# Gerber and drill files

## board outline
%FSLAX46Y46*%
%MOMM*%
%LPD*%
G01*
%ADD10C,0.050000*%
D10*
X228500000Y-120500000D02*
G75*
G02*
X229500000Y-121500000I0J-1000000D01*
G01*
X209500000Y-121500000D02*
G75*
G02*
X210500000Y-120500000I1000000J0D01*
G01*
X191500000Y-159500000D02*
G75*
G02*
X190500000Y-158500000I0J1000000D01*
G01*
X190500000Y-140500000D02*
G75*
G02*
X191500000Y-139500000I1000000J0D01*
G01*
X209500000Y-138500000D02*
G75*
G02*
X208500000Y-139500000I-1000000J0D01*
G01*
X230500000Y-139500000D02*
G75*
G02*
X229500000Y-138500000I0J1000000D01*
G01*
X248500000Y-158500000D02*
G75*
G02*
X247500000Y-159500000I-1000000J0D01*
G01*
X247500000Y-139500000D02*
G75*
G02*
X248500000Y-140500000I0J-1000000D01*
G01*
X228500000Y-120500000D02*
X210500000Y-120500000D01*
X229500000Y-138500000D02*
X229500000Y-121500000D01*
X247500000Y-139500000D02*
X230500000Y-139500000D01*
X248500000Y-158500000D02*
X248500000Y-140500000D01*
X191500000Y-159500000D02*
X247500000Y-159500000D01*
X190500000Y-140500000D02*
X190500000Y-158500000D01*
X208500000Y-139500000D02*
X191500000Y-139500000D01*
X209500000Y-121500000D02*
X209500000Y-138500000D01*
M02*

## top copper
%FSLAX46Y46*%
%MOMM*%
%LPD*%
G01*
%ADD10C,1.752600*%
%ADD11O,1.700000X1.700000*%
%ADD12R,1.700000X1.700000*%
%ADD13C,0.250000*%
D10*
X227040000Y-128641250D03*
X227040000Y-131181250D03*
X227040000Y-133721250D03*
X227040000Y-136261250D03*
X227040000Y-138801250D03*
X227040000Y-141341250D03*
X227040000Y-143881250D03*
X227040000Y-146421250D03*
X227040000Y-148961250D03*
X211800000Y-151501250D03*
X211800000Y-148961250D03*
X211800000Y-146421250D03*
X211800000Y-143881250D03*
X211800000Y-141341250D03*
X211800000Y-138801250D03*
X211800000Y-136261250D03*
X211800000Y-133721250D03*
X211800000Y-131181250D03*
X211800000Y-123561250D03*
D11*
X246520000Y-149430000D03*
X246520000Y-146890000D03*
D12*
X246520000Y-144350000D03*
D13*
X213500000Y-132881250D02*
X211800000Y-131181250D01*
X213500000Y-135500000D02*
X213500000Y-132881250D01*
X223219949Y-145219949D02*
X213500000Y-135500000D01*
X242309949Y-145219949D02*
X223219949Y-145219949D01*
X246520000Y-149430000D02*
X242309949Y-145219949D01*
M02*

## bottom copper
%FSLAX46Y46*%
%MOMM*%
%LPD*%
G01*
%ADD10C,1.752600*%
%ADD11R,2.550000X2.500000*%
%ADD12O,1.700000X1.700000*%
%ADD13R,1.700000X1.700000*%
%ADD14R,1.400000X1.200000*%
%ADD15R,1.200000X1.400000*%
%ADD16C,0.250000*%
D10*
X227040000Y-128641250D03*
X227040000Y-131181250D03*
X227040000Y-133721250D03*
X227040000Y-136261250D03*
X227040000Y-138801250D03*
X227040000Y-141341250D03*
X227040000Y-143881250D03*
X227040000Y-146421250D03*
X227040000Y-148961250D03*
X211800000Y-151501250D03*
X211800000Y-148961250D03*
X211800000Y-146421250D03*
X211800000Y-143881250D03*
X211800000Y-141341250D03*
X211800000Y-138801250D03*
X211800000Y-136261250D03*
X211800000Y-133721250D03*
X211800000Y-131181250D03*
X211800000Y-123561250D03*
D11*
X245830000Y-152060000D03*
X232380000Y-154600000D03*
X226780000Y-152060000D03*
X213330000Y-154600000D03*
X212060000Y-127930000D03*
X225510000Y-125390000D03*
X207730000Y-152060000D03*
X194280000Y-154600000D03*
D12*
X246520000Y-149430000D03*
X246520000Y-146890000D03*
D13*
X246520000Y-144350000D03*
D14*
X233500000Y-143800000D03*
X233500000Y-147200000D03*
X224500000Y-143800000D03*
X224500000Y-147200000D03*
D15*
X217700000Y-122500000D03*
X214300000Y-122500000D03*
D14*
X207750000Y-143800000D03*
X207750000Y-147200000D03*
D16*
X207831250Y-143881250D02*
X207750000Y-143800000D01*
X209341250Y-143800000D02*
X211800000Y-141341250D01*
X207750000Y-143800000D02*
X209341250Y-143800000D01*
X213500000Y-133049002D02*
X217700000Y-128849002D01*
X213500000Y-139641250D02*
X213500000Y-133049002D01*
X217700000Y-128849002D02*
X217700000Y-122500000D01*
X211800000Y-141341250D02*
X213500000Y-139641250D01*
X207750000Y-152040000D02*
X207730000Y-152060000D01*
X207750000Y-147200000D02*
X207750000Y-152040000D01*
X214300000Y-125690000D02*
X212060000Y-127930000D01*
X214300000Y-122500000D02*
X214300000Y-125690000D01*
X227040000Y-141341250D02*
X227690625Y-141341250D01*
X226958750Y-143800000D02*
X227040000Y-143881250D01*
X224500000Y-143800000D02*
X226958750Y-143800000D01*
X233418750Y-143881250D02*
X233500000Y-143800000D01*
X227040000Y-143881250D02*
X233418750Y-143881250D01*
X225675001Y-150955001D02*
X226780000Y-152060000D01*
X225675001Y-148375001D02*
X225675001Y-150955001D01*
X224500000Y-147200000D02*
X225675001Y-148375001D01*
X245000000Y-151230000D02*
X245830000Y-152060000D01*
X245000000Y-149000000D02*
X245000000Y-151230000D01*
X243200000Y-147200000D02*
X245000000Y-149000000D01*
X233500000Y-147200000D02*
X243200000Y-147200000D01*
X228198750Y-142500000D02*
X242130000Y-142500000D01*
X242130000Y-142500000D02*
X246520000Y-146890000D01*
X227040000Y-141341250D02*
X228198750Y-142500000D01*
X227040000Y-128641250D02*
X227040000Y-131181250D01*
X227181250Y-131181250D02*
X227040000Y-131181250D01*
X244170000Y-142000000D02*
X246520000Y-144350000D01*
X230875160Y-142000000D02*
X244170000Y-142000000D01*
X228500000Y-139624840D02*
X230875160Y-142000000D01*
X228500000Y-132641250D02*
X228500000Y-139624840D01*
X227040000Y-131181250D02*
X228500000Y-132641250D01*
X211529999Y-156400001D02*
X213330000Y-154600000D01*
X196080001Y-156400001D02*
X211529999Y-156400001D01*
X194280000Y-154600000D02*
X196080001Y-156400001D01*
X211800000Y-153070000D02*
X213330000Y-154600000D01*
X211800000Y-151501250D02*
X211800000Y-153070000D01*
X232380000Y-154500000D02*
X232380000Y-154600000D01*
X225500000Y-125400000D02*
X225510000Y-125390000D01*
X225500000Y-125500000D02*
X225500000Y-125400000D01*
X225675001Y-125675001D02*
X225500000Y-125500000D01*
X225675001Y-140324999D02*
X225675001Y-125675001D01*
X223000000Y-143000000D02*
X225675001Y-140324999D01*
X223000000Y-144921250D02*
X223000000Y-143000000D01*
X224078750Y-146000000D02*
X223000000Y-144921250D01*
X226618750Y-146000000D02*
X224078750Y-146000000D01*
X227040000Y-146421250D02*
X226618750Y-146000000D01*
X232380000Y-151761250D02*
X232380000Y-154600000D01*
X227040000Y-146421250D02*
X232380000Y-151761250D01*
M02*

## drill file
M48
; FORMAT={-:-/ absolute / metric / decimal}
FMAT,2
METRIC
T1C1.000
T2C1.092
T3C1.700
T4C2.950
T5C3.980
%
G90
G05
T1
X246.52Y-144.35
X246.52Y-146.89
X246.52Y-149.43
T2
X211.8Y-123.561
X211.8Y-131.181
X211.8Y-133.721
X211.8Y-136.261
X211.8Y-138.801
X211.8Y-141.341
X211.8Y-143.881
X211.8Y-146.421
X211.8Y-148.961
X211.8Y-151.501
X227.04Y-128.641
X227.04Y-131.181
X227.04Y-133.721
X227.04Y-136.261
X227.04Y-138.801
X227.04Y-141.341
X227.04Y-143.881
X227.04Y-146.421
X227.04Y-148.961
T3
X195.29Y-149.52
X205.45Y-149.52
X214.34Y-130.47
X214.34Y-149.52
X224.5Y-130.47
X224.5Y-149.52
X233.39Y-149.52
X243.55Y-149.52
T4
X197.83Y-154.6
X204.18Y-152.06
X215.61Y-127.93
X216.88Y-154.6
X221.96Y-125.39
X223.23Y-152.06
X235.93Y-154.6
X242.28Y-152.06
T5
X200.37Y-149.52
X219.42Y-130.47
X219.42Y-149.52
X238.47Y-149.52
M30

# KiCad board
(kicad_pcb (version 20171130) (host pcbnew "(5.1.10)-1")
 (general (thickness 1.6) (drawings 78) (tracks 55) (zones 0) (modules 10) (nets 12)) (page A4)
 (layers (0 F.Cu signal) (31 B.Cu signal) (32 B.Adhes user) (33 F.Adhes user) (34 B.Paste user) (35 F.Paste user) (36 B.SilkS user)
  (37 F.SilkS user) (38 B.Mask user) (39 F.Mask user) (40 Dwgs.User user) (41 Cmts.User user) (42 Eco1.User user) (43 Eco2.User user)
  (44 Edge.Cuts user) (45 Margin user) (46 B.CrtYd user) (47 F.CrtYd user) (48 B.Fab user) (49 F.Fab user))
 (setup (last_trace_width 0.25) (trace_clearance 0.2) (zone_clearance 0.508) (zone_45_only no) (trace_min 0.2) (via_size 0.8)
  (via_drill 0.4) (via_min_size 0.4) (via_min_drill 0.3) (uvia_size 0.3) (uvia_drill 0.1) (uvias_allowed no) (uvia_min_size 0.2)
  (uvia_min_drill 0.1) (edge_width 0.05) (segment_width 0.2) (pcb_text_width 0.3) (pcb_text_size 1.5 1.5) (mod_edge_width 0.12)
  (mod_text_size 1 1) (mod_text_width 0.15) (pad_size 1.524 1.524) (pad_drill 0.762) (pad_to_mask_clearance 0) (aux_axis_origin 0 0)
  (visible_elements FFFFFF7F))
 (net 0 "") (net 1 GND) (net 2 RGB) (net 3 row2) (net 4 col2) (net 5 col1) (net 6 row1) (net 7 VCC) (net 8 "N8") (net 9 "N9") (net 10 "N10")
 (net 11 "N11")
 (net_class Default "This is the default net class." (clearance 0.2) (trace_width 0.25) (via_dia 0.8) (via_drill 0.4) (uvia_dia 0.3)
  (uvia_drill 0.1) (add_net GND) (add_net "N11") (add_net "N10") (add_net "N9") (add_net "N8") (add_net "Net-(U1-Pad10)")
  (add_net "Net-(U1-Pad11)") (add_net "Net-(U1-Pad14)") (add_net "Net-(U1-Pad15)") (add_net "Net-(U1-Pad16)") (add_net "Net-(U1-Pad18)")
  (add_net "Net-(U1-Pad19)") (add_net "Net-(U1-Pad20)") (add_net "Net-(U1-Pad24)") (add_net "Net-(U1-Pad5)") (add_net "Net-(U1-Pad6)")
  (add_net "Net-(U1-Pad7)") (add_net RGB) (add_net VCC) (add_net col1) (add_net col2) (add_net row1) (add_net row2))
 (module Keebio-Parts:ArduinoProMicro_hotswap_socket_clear (layer B.Cu) (at 219.42 137.53125 270)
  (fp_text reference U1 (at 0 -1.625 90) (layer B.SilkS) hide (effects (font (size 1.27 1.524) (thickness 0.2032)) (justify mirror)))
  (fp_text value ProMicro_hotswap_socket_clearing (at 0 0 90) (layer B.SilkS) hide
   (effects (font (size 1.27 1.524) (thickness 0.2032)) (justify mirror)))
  (pad 3 thru_hole circle (at -8.89 -7.62 270) (size 1.7526 1.7526) (drill 1.0922) (layers *.Cu *.SilkS *.Mask) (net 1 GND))
  (pad 4 thru_hole circle (at -6.35 -7.62 270) (size 1.7526 1.7526) (drill 1.0922) (layers *.Cu *.SilkS *.Mask) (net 1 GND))
  (pad 5 thru_hole circle (at -3.81 -7.62 270) (size 1.7526 1.7526) (drill 1.0922) (layers *.Cu *.SilkS *.Mask))
  (pad 6 thru_hole circle (at -1.27 -7.62 270) (size 1.7526 1.7526) (drill 1.0922) (layers *.Cu *.SilkS *.Mask))
  (pad 7 thru_hole circle (at 1.27 -7.62 270) (size 1.7526 1.7526) (drill 1.0922) (layers *.Cu *.SilkS *.Mask))
  (pad 8 thru_hole circle (at 3.81 -7.62 270) (size 1.7526 1.7526) (drill 1.0922) (layers *.Cu *.SilkS *.Mask) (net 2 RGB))
  (pad 9 thru_hole circle (at 6.35 -7.62 270) (size 1.7526 1.7526) (drill 1.0922) (layers *.Cu *.SilkS *.Mask) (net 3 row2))
  (pad 10 thru_hole circle (at 8.89 -7.62 270) (size 1.7526 1.7526) (drill 1.0922) (layers *.Cu *.SilkS *.Mask) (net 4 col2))
  (pad 11 thru_hole circle (at 11.43 -7.62 270) (size 1.7526 1.7526) (drill 1.0922) (layers *.Cu *.SilkS *.Mask))
  (pad 13 thru_hole circle (at 13.97 7.62 270) (size 1.7526 1.7526) (drill 1.0922) (layers *.Cu *.SilkS *.Mask) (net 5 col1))
  (pad 14 thru_hole circle (at 11.43 7.62 270) (size 1.7526 1.7526) (drill 1.0922) (layers *.Cu *.SilkS *.Mask))
  (pad 15 thru_hole circle (at 8.89 7.62 270) (size 1.7526 1.7526) (drill 1.0922) (layers *.Cu *.SilkS *.Mask))
  (pad 16 thru_hole circle (at 6.35 7.62 270) (size 1.7526 1.7526) (drill 1.0922) (layers *.Cu *.SilkS *.Mask))
  (pad 17 thru_hole circle (at 3.81 7.62 270) (size 1.7526 1.7526) (drill 1.0922) (layers *.Cu *.SilkS *.Mask) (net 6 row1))
  (pad 18 thru_hole circle (at 1.27 7.62 270) (size 1.7526 1.7526) (drill 1.0922) (layers *.Cu *.SilkS *.Mask))
  (pad 19 thru_hole circle (at -1.27 7.62 270) (size 1.7526 1.7526) (drill 1.0922) (layers *.Cu *.SilkS *.Mask))
  (pad 20 thru_hole circle (at -3.81 7.62 270) (size 1.7526 1.7526) (drill 1.0922) (layers *.Cu *.SilkS *.Mask))
  (pad 21 thru_hole circle (at -6.35 7.62 270) (size 1.7526 1.7526) (drill 1.0922) (layers *.Cu *.SilkS *.Mask) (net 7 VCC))
  (pad 24 thru_hole circle (at -13.97 7.62 270) (size 1.7526 1.7526) (drill 1.0922) (layers *.Cu *.SilkS *.Mask)))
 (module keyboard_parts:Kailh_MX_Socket (layer F.Cu) (at 238.47 149.52)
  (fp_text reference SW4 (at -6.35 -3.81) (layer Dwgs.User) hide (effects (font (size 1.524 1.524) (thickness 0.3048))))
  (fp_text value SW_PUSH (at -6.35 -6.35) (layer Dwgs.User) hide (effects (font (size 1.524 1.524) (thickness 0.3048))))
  (pad 1 smd rect (at 7.36 2.54) (size 2.55 2.5) (layers B.Cu B.Paste B.Mask) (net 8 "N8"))
  (pad "" np_thru_hole circle (at 0 0) (size 3.98018 3.98018) (drill 3.98018) (layers *.Cu *.Mask))
  (pad "" np_thru_hole circle (at -2.54 5.08) (size 2.95 2.95) (drill 2.95) (layers *.Cu *.Mask))
  (pad "" np_thru_hole circle (at 3.81 2.54) (size 2.95 2.95) (drill 2.95) (layers *.Cu *.Mask))
  (pad 2 smd rect (at -6.09 5.08) (size 2.55 2.5) (layers B.Cu B.Paste B.Mask) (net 4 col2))
  (pad "" np_thru_hole circle (at -5.08 0) (size 1.7 1.7) (drill 1.7) (layers *.Cu *.Mask))
  (pad "" np_thru_hole circle (at 5.08 0) (size 1.7 1.7) (drill 1.7) (layers *.Cu *.Mask)))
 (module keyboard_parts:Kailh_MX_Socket (layer F.Cu) (at 219.42 149.52)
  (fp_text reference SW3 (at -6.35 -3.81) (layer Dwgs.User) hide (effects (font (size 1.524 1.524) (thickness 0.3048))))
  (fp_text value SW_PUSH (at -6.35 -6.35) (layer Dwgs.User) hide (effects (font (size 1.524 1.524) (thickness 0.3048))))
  (pad 1 smd rect (at 7.36 2.54) (size 2.55 2.5) (layers B.Cu B.Paste B.Mask) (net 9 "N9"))
  (pad "" np_thru_hole circle (at 0 0) (size 3.98018 3.98018) (drill 3.98018) (layers *.Cu *.Mask))
  (pad "" np_thru_hole circle (at -2.54 5.08) (size 2.95 2.95) (drill 2.95) (layers *.Cu *.Mask))
  (pad "" np_thru_hole circle (at 3.81 2.54) (size 2.95 2.95) (drill 2.95) (layers *.Cu *.Mask))
  (pad 2 smd rect (at -6.09 5.08) (size 2.55 2.5) (layers B.Cu B.Paste B.Mask) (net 5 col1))
  (pad "" np_thru_hole circle (at -5.08 0) (size 1.7 1.7) (drill 1.7) (layers *.Cu *.Mask))
  (pad "" np_thru_hole circle (at 5.08 0) (size 1.7 1.7) (drill 1.7) (layers *.Cu *.Mask)))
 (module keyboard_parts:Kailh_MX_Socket (layer F.Cu) (at 219.42 130.47 180)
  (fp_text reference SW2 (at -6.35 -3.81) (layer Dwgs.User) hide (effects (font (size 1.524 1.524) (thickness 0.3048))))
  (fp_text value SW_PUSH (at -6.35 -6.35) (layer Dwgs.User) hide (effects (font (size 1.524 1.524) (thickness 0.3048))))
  (pad 1 smd rect (at 7.36 2.54 180) (size 2.55 2.5) (layers B.Cu B.Paste B.Mask) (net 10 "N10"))
  (pad "" np_thru_hole circle (at 0 0 180) (size 3.98018 3.98018) (drill 3.98018) (layers *.Cu *.Mask))
  (pad "" np_thru_hole circle (at -2.54 5.08 180) (size 2.95 2.95) (drill 2.95) (layers *.Cu *.Mask))
  (pad "" np_thru_hole circle (at 3.81 2.54 180) (size 2.95 2.95) (drill 2.95) (layers *.Cu *.Mask))
  (pad 2 smd rect (at -6.09 5.08 180) (size 2.55 2.5) (layers B.Cu B.Paste B.Mask) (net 4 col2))
  (pad "" np_thru_hole circle (at -5.08 0 180) (size 1.7 1.7) (drill 1.7) (layers *.Cu *.Mask))
  (pad "" np_thru_hole circle (at 5.08 0 180) (size 1.7 1.7) (drill 1.7) (layers *.Cu *.Mask)))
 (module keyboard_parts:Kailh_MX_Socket (layer F.Cu) (at 200.37 149.52)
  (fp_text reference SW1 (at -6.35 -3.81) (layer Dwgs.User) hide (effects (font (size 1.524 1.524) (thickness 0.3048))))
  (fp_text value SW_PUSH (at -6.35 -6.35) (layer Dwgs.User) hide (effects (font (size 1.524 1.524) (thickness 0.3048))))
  (pad 1 smd rect (at 7.36 2.54) (size 2.55 2.5) (layers B.Cu B.Paste B.Mask) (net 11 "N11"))
  (pad "" np_thru_hole circle (at 0 0) (size 3.98018 3.98018) (drill 3.98018) (layers *.Cu *.Mask))
  (pad "" np_thru_hole circle (at -2.54 5.08) (size 2.95 2.95) (drill 2.95) (layers *.Cu *.Mask))
  (pad "" np_thru_hole circle (at 3.81 2.54) (size 2.95 2.95) (drill 2.95) (layers *.Cu *.Mask))
  (pad 2 smd rect (at -6.09 5.08) (size 2.55 2.5) (layers B.Cu B.Paste B.Mask) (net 5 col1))
  (pad "" np_thru_hole circle (at -5.08 0) (size 1.7 1.7) (drill 1.7) (layers *.Cu *.Mask))
  (pad "" np_thru_hole circle (at 5.08 0) (size 1.7 1.7) (drill 1.7) (layers *.Cu *.Mask)))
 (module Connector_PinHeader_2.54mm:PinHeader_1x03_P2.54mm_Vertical (layer F.Cu) (at 246.52 144.35)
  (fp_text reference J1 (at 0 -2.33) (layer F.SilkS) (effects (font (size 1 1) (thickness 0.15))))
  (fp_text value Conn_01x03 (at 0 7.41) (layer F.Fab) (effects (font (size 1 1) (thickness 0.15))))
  (pad 3 thru_hole oval (at 0 5.08) (size 1.7 1.7) (drill 1) (layers *.Cu *.Mask) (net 7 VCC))
  (pad 2 thru_hole oval (at 0 2.54) (size 1.7 1.7) (drill 1) (layers *.Cu *.Mask) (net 2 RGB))
  (pad 1 thru_hole rect (at 0 0) (size 1.7 1.7) (drill 1) (layers *.Cu *.Mask) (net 1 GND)))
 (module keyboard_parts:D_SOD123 (layer B.Cu) (at 233.5 145.5 270)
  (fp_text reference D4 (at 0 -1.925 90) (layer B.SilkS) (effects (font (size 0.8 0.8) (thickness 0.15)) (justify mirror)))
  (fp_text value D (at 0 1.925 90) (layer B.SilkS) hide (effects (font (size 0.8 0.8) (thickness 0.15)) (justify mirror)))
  (pad 1 smd rect (at -1.7 0 270) (size 1.2 1.4) (layers B.Cu B.Paste B.Mask) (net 3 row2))
  (pad 2 smd rect (at 1.7 0 270) (size 1.2 1.4) (layers B.Cu B.Paste B.Mask) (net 8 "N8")))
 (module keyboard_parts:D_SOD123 (layer B.Cu) (at 224.5 145.5 270)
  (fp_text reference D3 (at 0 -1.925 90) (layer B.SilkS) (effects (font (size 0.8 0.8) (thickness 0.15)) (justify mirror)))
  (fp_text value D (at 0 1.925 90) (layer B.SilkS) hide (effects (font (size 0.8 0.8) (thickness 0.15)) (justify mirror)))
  (pad 1 smd rect (at -1.7 0 270) (size 1.2 1.4) (layers B.Cu B.Paste B.Mask) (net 3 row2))
  (pad 2 smd rect (at 1.7 0 270) (size 1.2 1.4) (layers B.Cu B.Paste B.Mask) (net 9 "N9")))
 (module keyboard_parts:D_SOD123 (layer B.Cu) (at 216 122.5 180)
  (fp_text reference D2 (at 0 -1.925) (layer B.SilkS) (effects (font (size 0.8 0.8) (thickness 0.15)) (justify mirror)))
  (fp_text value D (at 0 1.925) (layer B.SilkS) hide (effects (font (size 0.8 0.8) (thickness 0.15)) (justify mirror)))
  (pad 1 smd rect (at -1.7 0 180) (size 1.2 1.4) (layers B.Cu B.Paste B.Mask) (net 6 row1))
  (pad 2 smd rect (at 1.7 0 180) (size 1.2 1.4) (layers B.Cu B.Paste B.Mask) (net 10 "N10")))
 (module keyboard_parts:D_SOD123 (layer B.Cu) (at 207.75 145.5 270)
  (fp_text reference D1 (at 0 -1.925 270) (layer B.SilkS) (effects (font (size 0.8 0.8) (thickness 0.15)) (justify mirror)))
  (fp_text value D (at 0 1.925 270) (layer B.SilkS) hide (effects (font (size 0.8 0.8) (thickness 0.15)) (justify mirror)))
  (pad 1 smd rect (at -1.7 0 270) (size 1.2 1.4) (layers B.Cu B.Paste B.Mask) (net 6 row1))
  (pad 2 smd rect (at 1.7 0 270) (size 1.2 1.4) (layers B.Cu B.Paste B.Mask) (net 11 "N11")))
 (gr_arc (start 228.5 121.5) (end 229.5 121.5) (angle -90) (layer Edge.Cuts) (width 0.05))
 (gr_arc (start 210.5 121.5) (end 210.5 120.5) (angle -90) (layer Edge.Cuts) (width 0.05))
 (gr_arc (start 191.5 158.5) (end 190.5 158.5) (angle -90) (layer Edge.Cuts) (width 0.05))
 (gr_arc (start 191.5 140.5) (end 191.5 139.5) (angle -90) (layer Edge.Cuts) (width 0.05))
 (gr_arc (start 208.5 138.5) (end 208.5 139.5) (angle -90) (layer Edge.Cuts) (width 0.05))
 (gr_arc (start 230.5 138.5) (end 229.5 138.5) (angle -90) (layer Edge.Cuts) (width 0.05))
 (gr_arc (start 247.5 158.5) (end 247.5 159.5) (angle -90) (layer Edge.Cuts) (width 0.05))
 (gr_arc (start 247.5 140.5) (end 248.5 140.5) (angle -90) (layer Edge.Cuts) (width 0.05))
 (gr_line (start 228.5 120.5) (end 210.5 120.5) (layer Edge.Cuts) (width 0.05))
 (gr_line (start 229.5 138.5) (end 229.5 121.5) (layer Edge.Cuts) (width 0.05))
 (gr_line (start 247.5 139.5) (end 230.5 139.5) (layer Edge.Cuts) (width 0.05))
 (gr_line (start 248.5 158.5) (end 248.5 140.5) (layer Edge.Cuts) (width 0.05))
 (gr_line (start 191.5 159.5) (end 247.5 159.5) (layer Edge.Cuts) (width 0.05))
 (gr_line (start 190.5 140.5) (end 190.5 158.5) (layer Edge.Cuts) (width 0.05))
 (gr_line (start 208.5 139.5) (end 191.5 139.5) (layer Edge.Cuts) (width 0.05))
 (gr_line (start 209.5 121.5) (end 209.5 138.5) (layer Edge.Cuts) (width 0.05))
 (segment (start 207.83125 143.88125) (end 207.75 143.8) (width 0.25) (layer B.Cu) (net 6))
 (segment (start 209.34125 143.8) (end 211.8 141.34125) (width 0.25) (layer B.Cu) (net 6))
 (segment (start 207.75 143.8) (end 209.34125 143.8) (width 0.25) (layer B.Cu) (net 6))
 (segment (start 213.5 133.049002) (end 217.7 128.849002) (width 0.25) (layer B.Cu) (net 6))
 (segment (start 213.5 139.64125) (end 213.5 133.049002) (width 0.25) (layer B.Cu) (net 6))
 (segment (start 217.7 128.849002) (end 217.7 122.5) (width 0.25) (layer B.Cu) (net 6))
 (segment (start 211.8 141.34125) (end 213.5 139.64125) (width 0.25) (layer B.Cu) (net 6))
 (segment (start 207.75 152.04) (end 207.73 152.06) (width 0.25) (layer B.Cu) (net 11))
 (segment (start 207.75 147.2) (end 207.75 152.04) (width 0.25) (layer B.Cu) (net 11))
 (segment (start 214.3 125.69) (end 212.06 127.93) (width 0.25) (layer B.Cu) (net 10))
 (segment (start 214.3 122.5) (end 214.3 125.69) (width 0.25) (layer B.Cu) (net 10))
 (segment (start 227.04 141.34125) (end 227.690625 141.34125) (width 0.25) (layer B.Cu) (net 2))
 (segment (start 226.95875 143.8) (end 227.04 143.88125) (width 0.25) (layer B.Cu) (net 3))
 (segment (start 224.5 143.8) (end 226.95875 143.8) (width 0.25) (layer B.Cu) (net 3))
 (segment (start 233.41875 143.88125) (end 233.5 143.8) (width 0.25) (layer B.Cu) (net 3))
 (segment (start 227.04 143.88125) (end 233.41875 143.88125) (width 0.25) (layer B.Cu) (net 3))
 (segment (start 225.675001 150.955001) (end 226.78 152.06) (width 0.25) (layer B.Cu) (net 9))
 (segment (start 225.675001 148.375001) (end 225.675001 150.955001) (width 0.25) (layer B.Cu) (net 9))
 (segment (start 224.5 147.2) (end 225.675001 148.375001) (width 0.25) (layer B.Cu) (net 9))
 (segment (start 245 151.23) (end 245.83 152.06) (width 0.25) (layer B.Cu) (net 8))
 (segment (start 245 149) (end 245 151.23) (width 0.25) (layer B.Cu) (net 8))
 (segment (start 243.2 147.2) (end 245 149) (width 0.25) (layer B.Cu) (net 8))
 (segment (start 233.5 147.2) (end 243.2 147.2) (width 0.25) (layer B.Cu) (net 8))
 (segment (start 213.5 132.88125) (end 211.8 131.18125) (width 0.25) (layer F.Cu) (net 7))
 (segment (start 213.5 135.5) (end 213.5 132.88125) (width 0.25) (layer F.Cu) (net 7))
 (segment (start 223.219949 145.219949) (end 213.5 135.5) (width 0.25) (layer F.Cu) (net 7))
 (segment (start 242.309949 145.219949) (end 223.219949 145.219949) (width 0.25) (layer F.Cu) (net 7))
 (segment (start 246.52 149.43) (end 242.309949 145.219949) (width 0.25) (layer F.Cu) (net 7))
 (segment (start 228.19875 142.5) (end 242.13 142.5) (width 0.25) (layer B.Cu) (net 2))
 (segment (start 242.13 142.5) (end 246.52 146.89) (width 0.25) (layer B.Cu) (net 2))
 (segment (start 227.04 141.34125) (end 228.19875 142.5) (width 0.25) (layer B.Cu) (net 2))
 (segment (start 227.04 128.64125) (end 227.04 131.18125) (width 0.25) (layer B.Cu) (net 1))
 (segment (start 227.18125 131.18125) (end 227.04 131.18125) (width 0.25) (layer B.Cu) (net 1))
 (segment (start 244.17 142) (end 246.52 144.35) (width 0.25) (layer B.Cu) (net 1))
 (segment (start 230.87516 142) (end 244.17 142) (width 0.25) (layer B.Cu) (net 1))
 (segment (start 228.5 139.62484) (end 230.87516 142) (width 0.25) (layer B.Cu) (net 1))
 (segment (start 228.5 132.64125) (end 228.5 139.62484) (width 0.25) (layer B.Cu) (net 1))
 (segment (start 227.04 131.18125) (end 228.5 132.64125) (width 0.25) (layer B.Cu) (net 1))
 (segment (start 211.529999 156.400001) (end 213.33 154.6) (width 0.25) (layer B.Cu) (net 5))
 (segment (start 196.080001 156.400001) (end 211.529999 156.400001) (width 0.25) (layer B.Cu) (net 5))
 (segment (start 194.28 154.6) (end 196.080001 156.400001) (width 0.25) (layer B.Cu) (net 5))
 (segment (start 211.8 153.07) (end 213.33 154.6) (width 0.25) (layer B.Cu) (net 5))
 (segment (start 211.8 151.50125) (end 211.8 153.07) (width 0.25) (layer B.Cu) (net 5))
 (segment (start 232.38 154.5) (end 232.38 154.6) (width 0.25) (layer B.Cu) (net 4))
 (segment (start 225.5 125.4) (end 225.51 125.39) (width 0.25) (layer B.Cu) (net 4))
 (segment (start 225.5 125.5) (end 225.5 125.4) (width 0.25) (layer B.Cu) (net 4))
 (segment (start 225.675001 125.675001) (end 225.5 125.5) (width 0.25) (layer B.Cu) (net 4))
 (segment (start 225.675001 140.324999) (end 225.675001 125.675001) (width 0.25) (layer B.Cu) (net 4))
 (segment (start 223 143) (end 225.675001 140.324999) (width 0.25) (layer B.Cu) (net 4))
 (segment (start 223 144.92125) (end 223 143) (width 0.25) (layer B.Cu) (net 4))
 (segment (start 224.07875 146) (end 223 144.92125) (width 0.25) (layer B.Cu) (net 4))
 (segment (start 226.61875 146) (end 224.07875 146) (width 0.25) (layer B.Cu) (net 4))
 (segment (start 227.04 146.42125) (end 226.61875 146) (width 0.25) (layer B.Cu) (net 4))
 (segment (start 232.38 151.76125) (end 232.38 154.6) (width 0.25) (layer B.Cu) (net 4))
 (segment (start 227.04 146.42125) (end 232.38 151.76125) (width 0.25) (layer B.Cu) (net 4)))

